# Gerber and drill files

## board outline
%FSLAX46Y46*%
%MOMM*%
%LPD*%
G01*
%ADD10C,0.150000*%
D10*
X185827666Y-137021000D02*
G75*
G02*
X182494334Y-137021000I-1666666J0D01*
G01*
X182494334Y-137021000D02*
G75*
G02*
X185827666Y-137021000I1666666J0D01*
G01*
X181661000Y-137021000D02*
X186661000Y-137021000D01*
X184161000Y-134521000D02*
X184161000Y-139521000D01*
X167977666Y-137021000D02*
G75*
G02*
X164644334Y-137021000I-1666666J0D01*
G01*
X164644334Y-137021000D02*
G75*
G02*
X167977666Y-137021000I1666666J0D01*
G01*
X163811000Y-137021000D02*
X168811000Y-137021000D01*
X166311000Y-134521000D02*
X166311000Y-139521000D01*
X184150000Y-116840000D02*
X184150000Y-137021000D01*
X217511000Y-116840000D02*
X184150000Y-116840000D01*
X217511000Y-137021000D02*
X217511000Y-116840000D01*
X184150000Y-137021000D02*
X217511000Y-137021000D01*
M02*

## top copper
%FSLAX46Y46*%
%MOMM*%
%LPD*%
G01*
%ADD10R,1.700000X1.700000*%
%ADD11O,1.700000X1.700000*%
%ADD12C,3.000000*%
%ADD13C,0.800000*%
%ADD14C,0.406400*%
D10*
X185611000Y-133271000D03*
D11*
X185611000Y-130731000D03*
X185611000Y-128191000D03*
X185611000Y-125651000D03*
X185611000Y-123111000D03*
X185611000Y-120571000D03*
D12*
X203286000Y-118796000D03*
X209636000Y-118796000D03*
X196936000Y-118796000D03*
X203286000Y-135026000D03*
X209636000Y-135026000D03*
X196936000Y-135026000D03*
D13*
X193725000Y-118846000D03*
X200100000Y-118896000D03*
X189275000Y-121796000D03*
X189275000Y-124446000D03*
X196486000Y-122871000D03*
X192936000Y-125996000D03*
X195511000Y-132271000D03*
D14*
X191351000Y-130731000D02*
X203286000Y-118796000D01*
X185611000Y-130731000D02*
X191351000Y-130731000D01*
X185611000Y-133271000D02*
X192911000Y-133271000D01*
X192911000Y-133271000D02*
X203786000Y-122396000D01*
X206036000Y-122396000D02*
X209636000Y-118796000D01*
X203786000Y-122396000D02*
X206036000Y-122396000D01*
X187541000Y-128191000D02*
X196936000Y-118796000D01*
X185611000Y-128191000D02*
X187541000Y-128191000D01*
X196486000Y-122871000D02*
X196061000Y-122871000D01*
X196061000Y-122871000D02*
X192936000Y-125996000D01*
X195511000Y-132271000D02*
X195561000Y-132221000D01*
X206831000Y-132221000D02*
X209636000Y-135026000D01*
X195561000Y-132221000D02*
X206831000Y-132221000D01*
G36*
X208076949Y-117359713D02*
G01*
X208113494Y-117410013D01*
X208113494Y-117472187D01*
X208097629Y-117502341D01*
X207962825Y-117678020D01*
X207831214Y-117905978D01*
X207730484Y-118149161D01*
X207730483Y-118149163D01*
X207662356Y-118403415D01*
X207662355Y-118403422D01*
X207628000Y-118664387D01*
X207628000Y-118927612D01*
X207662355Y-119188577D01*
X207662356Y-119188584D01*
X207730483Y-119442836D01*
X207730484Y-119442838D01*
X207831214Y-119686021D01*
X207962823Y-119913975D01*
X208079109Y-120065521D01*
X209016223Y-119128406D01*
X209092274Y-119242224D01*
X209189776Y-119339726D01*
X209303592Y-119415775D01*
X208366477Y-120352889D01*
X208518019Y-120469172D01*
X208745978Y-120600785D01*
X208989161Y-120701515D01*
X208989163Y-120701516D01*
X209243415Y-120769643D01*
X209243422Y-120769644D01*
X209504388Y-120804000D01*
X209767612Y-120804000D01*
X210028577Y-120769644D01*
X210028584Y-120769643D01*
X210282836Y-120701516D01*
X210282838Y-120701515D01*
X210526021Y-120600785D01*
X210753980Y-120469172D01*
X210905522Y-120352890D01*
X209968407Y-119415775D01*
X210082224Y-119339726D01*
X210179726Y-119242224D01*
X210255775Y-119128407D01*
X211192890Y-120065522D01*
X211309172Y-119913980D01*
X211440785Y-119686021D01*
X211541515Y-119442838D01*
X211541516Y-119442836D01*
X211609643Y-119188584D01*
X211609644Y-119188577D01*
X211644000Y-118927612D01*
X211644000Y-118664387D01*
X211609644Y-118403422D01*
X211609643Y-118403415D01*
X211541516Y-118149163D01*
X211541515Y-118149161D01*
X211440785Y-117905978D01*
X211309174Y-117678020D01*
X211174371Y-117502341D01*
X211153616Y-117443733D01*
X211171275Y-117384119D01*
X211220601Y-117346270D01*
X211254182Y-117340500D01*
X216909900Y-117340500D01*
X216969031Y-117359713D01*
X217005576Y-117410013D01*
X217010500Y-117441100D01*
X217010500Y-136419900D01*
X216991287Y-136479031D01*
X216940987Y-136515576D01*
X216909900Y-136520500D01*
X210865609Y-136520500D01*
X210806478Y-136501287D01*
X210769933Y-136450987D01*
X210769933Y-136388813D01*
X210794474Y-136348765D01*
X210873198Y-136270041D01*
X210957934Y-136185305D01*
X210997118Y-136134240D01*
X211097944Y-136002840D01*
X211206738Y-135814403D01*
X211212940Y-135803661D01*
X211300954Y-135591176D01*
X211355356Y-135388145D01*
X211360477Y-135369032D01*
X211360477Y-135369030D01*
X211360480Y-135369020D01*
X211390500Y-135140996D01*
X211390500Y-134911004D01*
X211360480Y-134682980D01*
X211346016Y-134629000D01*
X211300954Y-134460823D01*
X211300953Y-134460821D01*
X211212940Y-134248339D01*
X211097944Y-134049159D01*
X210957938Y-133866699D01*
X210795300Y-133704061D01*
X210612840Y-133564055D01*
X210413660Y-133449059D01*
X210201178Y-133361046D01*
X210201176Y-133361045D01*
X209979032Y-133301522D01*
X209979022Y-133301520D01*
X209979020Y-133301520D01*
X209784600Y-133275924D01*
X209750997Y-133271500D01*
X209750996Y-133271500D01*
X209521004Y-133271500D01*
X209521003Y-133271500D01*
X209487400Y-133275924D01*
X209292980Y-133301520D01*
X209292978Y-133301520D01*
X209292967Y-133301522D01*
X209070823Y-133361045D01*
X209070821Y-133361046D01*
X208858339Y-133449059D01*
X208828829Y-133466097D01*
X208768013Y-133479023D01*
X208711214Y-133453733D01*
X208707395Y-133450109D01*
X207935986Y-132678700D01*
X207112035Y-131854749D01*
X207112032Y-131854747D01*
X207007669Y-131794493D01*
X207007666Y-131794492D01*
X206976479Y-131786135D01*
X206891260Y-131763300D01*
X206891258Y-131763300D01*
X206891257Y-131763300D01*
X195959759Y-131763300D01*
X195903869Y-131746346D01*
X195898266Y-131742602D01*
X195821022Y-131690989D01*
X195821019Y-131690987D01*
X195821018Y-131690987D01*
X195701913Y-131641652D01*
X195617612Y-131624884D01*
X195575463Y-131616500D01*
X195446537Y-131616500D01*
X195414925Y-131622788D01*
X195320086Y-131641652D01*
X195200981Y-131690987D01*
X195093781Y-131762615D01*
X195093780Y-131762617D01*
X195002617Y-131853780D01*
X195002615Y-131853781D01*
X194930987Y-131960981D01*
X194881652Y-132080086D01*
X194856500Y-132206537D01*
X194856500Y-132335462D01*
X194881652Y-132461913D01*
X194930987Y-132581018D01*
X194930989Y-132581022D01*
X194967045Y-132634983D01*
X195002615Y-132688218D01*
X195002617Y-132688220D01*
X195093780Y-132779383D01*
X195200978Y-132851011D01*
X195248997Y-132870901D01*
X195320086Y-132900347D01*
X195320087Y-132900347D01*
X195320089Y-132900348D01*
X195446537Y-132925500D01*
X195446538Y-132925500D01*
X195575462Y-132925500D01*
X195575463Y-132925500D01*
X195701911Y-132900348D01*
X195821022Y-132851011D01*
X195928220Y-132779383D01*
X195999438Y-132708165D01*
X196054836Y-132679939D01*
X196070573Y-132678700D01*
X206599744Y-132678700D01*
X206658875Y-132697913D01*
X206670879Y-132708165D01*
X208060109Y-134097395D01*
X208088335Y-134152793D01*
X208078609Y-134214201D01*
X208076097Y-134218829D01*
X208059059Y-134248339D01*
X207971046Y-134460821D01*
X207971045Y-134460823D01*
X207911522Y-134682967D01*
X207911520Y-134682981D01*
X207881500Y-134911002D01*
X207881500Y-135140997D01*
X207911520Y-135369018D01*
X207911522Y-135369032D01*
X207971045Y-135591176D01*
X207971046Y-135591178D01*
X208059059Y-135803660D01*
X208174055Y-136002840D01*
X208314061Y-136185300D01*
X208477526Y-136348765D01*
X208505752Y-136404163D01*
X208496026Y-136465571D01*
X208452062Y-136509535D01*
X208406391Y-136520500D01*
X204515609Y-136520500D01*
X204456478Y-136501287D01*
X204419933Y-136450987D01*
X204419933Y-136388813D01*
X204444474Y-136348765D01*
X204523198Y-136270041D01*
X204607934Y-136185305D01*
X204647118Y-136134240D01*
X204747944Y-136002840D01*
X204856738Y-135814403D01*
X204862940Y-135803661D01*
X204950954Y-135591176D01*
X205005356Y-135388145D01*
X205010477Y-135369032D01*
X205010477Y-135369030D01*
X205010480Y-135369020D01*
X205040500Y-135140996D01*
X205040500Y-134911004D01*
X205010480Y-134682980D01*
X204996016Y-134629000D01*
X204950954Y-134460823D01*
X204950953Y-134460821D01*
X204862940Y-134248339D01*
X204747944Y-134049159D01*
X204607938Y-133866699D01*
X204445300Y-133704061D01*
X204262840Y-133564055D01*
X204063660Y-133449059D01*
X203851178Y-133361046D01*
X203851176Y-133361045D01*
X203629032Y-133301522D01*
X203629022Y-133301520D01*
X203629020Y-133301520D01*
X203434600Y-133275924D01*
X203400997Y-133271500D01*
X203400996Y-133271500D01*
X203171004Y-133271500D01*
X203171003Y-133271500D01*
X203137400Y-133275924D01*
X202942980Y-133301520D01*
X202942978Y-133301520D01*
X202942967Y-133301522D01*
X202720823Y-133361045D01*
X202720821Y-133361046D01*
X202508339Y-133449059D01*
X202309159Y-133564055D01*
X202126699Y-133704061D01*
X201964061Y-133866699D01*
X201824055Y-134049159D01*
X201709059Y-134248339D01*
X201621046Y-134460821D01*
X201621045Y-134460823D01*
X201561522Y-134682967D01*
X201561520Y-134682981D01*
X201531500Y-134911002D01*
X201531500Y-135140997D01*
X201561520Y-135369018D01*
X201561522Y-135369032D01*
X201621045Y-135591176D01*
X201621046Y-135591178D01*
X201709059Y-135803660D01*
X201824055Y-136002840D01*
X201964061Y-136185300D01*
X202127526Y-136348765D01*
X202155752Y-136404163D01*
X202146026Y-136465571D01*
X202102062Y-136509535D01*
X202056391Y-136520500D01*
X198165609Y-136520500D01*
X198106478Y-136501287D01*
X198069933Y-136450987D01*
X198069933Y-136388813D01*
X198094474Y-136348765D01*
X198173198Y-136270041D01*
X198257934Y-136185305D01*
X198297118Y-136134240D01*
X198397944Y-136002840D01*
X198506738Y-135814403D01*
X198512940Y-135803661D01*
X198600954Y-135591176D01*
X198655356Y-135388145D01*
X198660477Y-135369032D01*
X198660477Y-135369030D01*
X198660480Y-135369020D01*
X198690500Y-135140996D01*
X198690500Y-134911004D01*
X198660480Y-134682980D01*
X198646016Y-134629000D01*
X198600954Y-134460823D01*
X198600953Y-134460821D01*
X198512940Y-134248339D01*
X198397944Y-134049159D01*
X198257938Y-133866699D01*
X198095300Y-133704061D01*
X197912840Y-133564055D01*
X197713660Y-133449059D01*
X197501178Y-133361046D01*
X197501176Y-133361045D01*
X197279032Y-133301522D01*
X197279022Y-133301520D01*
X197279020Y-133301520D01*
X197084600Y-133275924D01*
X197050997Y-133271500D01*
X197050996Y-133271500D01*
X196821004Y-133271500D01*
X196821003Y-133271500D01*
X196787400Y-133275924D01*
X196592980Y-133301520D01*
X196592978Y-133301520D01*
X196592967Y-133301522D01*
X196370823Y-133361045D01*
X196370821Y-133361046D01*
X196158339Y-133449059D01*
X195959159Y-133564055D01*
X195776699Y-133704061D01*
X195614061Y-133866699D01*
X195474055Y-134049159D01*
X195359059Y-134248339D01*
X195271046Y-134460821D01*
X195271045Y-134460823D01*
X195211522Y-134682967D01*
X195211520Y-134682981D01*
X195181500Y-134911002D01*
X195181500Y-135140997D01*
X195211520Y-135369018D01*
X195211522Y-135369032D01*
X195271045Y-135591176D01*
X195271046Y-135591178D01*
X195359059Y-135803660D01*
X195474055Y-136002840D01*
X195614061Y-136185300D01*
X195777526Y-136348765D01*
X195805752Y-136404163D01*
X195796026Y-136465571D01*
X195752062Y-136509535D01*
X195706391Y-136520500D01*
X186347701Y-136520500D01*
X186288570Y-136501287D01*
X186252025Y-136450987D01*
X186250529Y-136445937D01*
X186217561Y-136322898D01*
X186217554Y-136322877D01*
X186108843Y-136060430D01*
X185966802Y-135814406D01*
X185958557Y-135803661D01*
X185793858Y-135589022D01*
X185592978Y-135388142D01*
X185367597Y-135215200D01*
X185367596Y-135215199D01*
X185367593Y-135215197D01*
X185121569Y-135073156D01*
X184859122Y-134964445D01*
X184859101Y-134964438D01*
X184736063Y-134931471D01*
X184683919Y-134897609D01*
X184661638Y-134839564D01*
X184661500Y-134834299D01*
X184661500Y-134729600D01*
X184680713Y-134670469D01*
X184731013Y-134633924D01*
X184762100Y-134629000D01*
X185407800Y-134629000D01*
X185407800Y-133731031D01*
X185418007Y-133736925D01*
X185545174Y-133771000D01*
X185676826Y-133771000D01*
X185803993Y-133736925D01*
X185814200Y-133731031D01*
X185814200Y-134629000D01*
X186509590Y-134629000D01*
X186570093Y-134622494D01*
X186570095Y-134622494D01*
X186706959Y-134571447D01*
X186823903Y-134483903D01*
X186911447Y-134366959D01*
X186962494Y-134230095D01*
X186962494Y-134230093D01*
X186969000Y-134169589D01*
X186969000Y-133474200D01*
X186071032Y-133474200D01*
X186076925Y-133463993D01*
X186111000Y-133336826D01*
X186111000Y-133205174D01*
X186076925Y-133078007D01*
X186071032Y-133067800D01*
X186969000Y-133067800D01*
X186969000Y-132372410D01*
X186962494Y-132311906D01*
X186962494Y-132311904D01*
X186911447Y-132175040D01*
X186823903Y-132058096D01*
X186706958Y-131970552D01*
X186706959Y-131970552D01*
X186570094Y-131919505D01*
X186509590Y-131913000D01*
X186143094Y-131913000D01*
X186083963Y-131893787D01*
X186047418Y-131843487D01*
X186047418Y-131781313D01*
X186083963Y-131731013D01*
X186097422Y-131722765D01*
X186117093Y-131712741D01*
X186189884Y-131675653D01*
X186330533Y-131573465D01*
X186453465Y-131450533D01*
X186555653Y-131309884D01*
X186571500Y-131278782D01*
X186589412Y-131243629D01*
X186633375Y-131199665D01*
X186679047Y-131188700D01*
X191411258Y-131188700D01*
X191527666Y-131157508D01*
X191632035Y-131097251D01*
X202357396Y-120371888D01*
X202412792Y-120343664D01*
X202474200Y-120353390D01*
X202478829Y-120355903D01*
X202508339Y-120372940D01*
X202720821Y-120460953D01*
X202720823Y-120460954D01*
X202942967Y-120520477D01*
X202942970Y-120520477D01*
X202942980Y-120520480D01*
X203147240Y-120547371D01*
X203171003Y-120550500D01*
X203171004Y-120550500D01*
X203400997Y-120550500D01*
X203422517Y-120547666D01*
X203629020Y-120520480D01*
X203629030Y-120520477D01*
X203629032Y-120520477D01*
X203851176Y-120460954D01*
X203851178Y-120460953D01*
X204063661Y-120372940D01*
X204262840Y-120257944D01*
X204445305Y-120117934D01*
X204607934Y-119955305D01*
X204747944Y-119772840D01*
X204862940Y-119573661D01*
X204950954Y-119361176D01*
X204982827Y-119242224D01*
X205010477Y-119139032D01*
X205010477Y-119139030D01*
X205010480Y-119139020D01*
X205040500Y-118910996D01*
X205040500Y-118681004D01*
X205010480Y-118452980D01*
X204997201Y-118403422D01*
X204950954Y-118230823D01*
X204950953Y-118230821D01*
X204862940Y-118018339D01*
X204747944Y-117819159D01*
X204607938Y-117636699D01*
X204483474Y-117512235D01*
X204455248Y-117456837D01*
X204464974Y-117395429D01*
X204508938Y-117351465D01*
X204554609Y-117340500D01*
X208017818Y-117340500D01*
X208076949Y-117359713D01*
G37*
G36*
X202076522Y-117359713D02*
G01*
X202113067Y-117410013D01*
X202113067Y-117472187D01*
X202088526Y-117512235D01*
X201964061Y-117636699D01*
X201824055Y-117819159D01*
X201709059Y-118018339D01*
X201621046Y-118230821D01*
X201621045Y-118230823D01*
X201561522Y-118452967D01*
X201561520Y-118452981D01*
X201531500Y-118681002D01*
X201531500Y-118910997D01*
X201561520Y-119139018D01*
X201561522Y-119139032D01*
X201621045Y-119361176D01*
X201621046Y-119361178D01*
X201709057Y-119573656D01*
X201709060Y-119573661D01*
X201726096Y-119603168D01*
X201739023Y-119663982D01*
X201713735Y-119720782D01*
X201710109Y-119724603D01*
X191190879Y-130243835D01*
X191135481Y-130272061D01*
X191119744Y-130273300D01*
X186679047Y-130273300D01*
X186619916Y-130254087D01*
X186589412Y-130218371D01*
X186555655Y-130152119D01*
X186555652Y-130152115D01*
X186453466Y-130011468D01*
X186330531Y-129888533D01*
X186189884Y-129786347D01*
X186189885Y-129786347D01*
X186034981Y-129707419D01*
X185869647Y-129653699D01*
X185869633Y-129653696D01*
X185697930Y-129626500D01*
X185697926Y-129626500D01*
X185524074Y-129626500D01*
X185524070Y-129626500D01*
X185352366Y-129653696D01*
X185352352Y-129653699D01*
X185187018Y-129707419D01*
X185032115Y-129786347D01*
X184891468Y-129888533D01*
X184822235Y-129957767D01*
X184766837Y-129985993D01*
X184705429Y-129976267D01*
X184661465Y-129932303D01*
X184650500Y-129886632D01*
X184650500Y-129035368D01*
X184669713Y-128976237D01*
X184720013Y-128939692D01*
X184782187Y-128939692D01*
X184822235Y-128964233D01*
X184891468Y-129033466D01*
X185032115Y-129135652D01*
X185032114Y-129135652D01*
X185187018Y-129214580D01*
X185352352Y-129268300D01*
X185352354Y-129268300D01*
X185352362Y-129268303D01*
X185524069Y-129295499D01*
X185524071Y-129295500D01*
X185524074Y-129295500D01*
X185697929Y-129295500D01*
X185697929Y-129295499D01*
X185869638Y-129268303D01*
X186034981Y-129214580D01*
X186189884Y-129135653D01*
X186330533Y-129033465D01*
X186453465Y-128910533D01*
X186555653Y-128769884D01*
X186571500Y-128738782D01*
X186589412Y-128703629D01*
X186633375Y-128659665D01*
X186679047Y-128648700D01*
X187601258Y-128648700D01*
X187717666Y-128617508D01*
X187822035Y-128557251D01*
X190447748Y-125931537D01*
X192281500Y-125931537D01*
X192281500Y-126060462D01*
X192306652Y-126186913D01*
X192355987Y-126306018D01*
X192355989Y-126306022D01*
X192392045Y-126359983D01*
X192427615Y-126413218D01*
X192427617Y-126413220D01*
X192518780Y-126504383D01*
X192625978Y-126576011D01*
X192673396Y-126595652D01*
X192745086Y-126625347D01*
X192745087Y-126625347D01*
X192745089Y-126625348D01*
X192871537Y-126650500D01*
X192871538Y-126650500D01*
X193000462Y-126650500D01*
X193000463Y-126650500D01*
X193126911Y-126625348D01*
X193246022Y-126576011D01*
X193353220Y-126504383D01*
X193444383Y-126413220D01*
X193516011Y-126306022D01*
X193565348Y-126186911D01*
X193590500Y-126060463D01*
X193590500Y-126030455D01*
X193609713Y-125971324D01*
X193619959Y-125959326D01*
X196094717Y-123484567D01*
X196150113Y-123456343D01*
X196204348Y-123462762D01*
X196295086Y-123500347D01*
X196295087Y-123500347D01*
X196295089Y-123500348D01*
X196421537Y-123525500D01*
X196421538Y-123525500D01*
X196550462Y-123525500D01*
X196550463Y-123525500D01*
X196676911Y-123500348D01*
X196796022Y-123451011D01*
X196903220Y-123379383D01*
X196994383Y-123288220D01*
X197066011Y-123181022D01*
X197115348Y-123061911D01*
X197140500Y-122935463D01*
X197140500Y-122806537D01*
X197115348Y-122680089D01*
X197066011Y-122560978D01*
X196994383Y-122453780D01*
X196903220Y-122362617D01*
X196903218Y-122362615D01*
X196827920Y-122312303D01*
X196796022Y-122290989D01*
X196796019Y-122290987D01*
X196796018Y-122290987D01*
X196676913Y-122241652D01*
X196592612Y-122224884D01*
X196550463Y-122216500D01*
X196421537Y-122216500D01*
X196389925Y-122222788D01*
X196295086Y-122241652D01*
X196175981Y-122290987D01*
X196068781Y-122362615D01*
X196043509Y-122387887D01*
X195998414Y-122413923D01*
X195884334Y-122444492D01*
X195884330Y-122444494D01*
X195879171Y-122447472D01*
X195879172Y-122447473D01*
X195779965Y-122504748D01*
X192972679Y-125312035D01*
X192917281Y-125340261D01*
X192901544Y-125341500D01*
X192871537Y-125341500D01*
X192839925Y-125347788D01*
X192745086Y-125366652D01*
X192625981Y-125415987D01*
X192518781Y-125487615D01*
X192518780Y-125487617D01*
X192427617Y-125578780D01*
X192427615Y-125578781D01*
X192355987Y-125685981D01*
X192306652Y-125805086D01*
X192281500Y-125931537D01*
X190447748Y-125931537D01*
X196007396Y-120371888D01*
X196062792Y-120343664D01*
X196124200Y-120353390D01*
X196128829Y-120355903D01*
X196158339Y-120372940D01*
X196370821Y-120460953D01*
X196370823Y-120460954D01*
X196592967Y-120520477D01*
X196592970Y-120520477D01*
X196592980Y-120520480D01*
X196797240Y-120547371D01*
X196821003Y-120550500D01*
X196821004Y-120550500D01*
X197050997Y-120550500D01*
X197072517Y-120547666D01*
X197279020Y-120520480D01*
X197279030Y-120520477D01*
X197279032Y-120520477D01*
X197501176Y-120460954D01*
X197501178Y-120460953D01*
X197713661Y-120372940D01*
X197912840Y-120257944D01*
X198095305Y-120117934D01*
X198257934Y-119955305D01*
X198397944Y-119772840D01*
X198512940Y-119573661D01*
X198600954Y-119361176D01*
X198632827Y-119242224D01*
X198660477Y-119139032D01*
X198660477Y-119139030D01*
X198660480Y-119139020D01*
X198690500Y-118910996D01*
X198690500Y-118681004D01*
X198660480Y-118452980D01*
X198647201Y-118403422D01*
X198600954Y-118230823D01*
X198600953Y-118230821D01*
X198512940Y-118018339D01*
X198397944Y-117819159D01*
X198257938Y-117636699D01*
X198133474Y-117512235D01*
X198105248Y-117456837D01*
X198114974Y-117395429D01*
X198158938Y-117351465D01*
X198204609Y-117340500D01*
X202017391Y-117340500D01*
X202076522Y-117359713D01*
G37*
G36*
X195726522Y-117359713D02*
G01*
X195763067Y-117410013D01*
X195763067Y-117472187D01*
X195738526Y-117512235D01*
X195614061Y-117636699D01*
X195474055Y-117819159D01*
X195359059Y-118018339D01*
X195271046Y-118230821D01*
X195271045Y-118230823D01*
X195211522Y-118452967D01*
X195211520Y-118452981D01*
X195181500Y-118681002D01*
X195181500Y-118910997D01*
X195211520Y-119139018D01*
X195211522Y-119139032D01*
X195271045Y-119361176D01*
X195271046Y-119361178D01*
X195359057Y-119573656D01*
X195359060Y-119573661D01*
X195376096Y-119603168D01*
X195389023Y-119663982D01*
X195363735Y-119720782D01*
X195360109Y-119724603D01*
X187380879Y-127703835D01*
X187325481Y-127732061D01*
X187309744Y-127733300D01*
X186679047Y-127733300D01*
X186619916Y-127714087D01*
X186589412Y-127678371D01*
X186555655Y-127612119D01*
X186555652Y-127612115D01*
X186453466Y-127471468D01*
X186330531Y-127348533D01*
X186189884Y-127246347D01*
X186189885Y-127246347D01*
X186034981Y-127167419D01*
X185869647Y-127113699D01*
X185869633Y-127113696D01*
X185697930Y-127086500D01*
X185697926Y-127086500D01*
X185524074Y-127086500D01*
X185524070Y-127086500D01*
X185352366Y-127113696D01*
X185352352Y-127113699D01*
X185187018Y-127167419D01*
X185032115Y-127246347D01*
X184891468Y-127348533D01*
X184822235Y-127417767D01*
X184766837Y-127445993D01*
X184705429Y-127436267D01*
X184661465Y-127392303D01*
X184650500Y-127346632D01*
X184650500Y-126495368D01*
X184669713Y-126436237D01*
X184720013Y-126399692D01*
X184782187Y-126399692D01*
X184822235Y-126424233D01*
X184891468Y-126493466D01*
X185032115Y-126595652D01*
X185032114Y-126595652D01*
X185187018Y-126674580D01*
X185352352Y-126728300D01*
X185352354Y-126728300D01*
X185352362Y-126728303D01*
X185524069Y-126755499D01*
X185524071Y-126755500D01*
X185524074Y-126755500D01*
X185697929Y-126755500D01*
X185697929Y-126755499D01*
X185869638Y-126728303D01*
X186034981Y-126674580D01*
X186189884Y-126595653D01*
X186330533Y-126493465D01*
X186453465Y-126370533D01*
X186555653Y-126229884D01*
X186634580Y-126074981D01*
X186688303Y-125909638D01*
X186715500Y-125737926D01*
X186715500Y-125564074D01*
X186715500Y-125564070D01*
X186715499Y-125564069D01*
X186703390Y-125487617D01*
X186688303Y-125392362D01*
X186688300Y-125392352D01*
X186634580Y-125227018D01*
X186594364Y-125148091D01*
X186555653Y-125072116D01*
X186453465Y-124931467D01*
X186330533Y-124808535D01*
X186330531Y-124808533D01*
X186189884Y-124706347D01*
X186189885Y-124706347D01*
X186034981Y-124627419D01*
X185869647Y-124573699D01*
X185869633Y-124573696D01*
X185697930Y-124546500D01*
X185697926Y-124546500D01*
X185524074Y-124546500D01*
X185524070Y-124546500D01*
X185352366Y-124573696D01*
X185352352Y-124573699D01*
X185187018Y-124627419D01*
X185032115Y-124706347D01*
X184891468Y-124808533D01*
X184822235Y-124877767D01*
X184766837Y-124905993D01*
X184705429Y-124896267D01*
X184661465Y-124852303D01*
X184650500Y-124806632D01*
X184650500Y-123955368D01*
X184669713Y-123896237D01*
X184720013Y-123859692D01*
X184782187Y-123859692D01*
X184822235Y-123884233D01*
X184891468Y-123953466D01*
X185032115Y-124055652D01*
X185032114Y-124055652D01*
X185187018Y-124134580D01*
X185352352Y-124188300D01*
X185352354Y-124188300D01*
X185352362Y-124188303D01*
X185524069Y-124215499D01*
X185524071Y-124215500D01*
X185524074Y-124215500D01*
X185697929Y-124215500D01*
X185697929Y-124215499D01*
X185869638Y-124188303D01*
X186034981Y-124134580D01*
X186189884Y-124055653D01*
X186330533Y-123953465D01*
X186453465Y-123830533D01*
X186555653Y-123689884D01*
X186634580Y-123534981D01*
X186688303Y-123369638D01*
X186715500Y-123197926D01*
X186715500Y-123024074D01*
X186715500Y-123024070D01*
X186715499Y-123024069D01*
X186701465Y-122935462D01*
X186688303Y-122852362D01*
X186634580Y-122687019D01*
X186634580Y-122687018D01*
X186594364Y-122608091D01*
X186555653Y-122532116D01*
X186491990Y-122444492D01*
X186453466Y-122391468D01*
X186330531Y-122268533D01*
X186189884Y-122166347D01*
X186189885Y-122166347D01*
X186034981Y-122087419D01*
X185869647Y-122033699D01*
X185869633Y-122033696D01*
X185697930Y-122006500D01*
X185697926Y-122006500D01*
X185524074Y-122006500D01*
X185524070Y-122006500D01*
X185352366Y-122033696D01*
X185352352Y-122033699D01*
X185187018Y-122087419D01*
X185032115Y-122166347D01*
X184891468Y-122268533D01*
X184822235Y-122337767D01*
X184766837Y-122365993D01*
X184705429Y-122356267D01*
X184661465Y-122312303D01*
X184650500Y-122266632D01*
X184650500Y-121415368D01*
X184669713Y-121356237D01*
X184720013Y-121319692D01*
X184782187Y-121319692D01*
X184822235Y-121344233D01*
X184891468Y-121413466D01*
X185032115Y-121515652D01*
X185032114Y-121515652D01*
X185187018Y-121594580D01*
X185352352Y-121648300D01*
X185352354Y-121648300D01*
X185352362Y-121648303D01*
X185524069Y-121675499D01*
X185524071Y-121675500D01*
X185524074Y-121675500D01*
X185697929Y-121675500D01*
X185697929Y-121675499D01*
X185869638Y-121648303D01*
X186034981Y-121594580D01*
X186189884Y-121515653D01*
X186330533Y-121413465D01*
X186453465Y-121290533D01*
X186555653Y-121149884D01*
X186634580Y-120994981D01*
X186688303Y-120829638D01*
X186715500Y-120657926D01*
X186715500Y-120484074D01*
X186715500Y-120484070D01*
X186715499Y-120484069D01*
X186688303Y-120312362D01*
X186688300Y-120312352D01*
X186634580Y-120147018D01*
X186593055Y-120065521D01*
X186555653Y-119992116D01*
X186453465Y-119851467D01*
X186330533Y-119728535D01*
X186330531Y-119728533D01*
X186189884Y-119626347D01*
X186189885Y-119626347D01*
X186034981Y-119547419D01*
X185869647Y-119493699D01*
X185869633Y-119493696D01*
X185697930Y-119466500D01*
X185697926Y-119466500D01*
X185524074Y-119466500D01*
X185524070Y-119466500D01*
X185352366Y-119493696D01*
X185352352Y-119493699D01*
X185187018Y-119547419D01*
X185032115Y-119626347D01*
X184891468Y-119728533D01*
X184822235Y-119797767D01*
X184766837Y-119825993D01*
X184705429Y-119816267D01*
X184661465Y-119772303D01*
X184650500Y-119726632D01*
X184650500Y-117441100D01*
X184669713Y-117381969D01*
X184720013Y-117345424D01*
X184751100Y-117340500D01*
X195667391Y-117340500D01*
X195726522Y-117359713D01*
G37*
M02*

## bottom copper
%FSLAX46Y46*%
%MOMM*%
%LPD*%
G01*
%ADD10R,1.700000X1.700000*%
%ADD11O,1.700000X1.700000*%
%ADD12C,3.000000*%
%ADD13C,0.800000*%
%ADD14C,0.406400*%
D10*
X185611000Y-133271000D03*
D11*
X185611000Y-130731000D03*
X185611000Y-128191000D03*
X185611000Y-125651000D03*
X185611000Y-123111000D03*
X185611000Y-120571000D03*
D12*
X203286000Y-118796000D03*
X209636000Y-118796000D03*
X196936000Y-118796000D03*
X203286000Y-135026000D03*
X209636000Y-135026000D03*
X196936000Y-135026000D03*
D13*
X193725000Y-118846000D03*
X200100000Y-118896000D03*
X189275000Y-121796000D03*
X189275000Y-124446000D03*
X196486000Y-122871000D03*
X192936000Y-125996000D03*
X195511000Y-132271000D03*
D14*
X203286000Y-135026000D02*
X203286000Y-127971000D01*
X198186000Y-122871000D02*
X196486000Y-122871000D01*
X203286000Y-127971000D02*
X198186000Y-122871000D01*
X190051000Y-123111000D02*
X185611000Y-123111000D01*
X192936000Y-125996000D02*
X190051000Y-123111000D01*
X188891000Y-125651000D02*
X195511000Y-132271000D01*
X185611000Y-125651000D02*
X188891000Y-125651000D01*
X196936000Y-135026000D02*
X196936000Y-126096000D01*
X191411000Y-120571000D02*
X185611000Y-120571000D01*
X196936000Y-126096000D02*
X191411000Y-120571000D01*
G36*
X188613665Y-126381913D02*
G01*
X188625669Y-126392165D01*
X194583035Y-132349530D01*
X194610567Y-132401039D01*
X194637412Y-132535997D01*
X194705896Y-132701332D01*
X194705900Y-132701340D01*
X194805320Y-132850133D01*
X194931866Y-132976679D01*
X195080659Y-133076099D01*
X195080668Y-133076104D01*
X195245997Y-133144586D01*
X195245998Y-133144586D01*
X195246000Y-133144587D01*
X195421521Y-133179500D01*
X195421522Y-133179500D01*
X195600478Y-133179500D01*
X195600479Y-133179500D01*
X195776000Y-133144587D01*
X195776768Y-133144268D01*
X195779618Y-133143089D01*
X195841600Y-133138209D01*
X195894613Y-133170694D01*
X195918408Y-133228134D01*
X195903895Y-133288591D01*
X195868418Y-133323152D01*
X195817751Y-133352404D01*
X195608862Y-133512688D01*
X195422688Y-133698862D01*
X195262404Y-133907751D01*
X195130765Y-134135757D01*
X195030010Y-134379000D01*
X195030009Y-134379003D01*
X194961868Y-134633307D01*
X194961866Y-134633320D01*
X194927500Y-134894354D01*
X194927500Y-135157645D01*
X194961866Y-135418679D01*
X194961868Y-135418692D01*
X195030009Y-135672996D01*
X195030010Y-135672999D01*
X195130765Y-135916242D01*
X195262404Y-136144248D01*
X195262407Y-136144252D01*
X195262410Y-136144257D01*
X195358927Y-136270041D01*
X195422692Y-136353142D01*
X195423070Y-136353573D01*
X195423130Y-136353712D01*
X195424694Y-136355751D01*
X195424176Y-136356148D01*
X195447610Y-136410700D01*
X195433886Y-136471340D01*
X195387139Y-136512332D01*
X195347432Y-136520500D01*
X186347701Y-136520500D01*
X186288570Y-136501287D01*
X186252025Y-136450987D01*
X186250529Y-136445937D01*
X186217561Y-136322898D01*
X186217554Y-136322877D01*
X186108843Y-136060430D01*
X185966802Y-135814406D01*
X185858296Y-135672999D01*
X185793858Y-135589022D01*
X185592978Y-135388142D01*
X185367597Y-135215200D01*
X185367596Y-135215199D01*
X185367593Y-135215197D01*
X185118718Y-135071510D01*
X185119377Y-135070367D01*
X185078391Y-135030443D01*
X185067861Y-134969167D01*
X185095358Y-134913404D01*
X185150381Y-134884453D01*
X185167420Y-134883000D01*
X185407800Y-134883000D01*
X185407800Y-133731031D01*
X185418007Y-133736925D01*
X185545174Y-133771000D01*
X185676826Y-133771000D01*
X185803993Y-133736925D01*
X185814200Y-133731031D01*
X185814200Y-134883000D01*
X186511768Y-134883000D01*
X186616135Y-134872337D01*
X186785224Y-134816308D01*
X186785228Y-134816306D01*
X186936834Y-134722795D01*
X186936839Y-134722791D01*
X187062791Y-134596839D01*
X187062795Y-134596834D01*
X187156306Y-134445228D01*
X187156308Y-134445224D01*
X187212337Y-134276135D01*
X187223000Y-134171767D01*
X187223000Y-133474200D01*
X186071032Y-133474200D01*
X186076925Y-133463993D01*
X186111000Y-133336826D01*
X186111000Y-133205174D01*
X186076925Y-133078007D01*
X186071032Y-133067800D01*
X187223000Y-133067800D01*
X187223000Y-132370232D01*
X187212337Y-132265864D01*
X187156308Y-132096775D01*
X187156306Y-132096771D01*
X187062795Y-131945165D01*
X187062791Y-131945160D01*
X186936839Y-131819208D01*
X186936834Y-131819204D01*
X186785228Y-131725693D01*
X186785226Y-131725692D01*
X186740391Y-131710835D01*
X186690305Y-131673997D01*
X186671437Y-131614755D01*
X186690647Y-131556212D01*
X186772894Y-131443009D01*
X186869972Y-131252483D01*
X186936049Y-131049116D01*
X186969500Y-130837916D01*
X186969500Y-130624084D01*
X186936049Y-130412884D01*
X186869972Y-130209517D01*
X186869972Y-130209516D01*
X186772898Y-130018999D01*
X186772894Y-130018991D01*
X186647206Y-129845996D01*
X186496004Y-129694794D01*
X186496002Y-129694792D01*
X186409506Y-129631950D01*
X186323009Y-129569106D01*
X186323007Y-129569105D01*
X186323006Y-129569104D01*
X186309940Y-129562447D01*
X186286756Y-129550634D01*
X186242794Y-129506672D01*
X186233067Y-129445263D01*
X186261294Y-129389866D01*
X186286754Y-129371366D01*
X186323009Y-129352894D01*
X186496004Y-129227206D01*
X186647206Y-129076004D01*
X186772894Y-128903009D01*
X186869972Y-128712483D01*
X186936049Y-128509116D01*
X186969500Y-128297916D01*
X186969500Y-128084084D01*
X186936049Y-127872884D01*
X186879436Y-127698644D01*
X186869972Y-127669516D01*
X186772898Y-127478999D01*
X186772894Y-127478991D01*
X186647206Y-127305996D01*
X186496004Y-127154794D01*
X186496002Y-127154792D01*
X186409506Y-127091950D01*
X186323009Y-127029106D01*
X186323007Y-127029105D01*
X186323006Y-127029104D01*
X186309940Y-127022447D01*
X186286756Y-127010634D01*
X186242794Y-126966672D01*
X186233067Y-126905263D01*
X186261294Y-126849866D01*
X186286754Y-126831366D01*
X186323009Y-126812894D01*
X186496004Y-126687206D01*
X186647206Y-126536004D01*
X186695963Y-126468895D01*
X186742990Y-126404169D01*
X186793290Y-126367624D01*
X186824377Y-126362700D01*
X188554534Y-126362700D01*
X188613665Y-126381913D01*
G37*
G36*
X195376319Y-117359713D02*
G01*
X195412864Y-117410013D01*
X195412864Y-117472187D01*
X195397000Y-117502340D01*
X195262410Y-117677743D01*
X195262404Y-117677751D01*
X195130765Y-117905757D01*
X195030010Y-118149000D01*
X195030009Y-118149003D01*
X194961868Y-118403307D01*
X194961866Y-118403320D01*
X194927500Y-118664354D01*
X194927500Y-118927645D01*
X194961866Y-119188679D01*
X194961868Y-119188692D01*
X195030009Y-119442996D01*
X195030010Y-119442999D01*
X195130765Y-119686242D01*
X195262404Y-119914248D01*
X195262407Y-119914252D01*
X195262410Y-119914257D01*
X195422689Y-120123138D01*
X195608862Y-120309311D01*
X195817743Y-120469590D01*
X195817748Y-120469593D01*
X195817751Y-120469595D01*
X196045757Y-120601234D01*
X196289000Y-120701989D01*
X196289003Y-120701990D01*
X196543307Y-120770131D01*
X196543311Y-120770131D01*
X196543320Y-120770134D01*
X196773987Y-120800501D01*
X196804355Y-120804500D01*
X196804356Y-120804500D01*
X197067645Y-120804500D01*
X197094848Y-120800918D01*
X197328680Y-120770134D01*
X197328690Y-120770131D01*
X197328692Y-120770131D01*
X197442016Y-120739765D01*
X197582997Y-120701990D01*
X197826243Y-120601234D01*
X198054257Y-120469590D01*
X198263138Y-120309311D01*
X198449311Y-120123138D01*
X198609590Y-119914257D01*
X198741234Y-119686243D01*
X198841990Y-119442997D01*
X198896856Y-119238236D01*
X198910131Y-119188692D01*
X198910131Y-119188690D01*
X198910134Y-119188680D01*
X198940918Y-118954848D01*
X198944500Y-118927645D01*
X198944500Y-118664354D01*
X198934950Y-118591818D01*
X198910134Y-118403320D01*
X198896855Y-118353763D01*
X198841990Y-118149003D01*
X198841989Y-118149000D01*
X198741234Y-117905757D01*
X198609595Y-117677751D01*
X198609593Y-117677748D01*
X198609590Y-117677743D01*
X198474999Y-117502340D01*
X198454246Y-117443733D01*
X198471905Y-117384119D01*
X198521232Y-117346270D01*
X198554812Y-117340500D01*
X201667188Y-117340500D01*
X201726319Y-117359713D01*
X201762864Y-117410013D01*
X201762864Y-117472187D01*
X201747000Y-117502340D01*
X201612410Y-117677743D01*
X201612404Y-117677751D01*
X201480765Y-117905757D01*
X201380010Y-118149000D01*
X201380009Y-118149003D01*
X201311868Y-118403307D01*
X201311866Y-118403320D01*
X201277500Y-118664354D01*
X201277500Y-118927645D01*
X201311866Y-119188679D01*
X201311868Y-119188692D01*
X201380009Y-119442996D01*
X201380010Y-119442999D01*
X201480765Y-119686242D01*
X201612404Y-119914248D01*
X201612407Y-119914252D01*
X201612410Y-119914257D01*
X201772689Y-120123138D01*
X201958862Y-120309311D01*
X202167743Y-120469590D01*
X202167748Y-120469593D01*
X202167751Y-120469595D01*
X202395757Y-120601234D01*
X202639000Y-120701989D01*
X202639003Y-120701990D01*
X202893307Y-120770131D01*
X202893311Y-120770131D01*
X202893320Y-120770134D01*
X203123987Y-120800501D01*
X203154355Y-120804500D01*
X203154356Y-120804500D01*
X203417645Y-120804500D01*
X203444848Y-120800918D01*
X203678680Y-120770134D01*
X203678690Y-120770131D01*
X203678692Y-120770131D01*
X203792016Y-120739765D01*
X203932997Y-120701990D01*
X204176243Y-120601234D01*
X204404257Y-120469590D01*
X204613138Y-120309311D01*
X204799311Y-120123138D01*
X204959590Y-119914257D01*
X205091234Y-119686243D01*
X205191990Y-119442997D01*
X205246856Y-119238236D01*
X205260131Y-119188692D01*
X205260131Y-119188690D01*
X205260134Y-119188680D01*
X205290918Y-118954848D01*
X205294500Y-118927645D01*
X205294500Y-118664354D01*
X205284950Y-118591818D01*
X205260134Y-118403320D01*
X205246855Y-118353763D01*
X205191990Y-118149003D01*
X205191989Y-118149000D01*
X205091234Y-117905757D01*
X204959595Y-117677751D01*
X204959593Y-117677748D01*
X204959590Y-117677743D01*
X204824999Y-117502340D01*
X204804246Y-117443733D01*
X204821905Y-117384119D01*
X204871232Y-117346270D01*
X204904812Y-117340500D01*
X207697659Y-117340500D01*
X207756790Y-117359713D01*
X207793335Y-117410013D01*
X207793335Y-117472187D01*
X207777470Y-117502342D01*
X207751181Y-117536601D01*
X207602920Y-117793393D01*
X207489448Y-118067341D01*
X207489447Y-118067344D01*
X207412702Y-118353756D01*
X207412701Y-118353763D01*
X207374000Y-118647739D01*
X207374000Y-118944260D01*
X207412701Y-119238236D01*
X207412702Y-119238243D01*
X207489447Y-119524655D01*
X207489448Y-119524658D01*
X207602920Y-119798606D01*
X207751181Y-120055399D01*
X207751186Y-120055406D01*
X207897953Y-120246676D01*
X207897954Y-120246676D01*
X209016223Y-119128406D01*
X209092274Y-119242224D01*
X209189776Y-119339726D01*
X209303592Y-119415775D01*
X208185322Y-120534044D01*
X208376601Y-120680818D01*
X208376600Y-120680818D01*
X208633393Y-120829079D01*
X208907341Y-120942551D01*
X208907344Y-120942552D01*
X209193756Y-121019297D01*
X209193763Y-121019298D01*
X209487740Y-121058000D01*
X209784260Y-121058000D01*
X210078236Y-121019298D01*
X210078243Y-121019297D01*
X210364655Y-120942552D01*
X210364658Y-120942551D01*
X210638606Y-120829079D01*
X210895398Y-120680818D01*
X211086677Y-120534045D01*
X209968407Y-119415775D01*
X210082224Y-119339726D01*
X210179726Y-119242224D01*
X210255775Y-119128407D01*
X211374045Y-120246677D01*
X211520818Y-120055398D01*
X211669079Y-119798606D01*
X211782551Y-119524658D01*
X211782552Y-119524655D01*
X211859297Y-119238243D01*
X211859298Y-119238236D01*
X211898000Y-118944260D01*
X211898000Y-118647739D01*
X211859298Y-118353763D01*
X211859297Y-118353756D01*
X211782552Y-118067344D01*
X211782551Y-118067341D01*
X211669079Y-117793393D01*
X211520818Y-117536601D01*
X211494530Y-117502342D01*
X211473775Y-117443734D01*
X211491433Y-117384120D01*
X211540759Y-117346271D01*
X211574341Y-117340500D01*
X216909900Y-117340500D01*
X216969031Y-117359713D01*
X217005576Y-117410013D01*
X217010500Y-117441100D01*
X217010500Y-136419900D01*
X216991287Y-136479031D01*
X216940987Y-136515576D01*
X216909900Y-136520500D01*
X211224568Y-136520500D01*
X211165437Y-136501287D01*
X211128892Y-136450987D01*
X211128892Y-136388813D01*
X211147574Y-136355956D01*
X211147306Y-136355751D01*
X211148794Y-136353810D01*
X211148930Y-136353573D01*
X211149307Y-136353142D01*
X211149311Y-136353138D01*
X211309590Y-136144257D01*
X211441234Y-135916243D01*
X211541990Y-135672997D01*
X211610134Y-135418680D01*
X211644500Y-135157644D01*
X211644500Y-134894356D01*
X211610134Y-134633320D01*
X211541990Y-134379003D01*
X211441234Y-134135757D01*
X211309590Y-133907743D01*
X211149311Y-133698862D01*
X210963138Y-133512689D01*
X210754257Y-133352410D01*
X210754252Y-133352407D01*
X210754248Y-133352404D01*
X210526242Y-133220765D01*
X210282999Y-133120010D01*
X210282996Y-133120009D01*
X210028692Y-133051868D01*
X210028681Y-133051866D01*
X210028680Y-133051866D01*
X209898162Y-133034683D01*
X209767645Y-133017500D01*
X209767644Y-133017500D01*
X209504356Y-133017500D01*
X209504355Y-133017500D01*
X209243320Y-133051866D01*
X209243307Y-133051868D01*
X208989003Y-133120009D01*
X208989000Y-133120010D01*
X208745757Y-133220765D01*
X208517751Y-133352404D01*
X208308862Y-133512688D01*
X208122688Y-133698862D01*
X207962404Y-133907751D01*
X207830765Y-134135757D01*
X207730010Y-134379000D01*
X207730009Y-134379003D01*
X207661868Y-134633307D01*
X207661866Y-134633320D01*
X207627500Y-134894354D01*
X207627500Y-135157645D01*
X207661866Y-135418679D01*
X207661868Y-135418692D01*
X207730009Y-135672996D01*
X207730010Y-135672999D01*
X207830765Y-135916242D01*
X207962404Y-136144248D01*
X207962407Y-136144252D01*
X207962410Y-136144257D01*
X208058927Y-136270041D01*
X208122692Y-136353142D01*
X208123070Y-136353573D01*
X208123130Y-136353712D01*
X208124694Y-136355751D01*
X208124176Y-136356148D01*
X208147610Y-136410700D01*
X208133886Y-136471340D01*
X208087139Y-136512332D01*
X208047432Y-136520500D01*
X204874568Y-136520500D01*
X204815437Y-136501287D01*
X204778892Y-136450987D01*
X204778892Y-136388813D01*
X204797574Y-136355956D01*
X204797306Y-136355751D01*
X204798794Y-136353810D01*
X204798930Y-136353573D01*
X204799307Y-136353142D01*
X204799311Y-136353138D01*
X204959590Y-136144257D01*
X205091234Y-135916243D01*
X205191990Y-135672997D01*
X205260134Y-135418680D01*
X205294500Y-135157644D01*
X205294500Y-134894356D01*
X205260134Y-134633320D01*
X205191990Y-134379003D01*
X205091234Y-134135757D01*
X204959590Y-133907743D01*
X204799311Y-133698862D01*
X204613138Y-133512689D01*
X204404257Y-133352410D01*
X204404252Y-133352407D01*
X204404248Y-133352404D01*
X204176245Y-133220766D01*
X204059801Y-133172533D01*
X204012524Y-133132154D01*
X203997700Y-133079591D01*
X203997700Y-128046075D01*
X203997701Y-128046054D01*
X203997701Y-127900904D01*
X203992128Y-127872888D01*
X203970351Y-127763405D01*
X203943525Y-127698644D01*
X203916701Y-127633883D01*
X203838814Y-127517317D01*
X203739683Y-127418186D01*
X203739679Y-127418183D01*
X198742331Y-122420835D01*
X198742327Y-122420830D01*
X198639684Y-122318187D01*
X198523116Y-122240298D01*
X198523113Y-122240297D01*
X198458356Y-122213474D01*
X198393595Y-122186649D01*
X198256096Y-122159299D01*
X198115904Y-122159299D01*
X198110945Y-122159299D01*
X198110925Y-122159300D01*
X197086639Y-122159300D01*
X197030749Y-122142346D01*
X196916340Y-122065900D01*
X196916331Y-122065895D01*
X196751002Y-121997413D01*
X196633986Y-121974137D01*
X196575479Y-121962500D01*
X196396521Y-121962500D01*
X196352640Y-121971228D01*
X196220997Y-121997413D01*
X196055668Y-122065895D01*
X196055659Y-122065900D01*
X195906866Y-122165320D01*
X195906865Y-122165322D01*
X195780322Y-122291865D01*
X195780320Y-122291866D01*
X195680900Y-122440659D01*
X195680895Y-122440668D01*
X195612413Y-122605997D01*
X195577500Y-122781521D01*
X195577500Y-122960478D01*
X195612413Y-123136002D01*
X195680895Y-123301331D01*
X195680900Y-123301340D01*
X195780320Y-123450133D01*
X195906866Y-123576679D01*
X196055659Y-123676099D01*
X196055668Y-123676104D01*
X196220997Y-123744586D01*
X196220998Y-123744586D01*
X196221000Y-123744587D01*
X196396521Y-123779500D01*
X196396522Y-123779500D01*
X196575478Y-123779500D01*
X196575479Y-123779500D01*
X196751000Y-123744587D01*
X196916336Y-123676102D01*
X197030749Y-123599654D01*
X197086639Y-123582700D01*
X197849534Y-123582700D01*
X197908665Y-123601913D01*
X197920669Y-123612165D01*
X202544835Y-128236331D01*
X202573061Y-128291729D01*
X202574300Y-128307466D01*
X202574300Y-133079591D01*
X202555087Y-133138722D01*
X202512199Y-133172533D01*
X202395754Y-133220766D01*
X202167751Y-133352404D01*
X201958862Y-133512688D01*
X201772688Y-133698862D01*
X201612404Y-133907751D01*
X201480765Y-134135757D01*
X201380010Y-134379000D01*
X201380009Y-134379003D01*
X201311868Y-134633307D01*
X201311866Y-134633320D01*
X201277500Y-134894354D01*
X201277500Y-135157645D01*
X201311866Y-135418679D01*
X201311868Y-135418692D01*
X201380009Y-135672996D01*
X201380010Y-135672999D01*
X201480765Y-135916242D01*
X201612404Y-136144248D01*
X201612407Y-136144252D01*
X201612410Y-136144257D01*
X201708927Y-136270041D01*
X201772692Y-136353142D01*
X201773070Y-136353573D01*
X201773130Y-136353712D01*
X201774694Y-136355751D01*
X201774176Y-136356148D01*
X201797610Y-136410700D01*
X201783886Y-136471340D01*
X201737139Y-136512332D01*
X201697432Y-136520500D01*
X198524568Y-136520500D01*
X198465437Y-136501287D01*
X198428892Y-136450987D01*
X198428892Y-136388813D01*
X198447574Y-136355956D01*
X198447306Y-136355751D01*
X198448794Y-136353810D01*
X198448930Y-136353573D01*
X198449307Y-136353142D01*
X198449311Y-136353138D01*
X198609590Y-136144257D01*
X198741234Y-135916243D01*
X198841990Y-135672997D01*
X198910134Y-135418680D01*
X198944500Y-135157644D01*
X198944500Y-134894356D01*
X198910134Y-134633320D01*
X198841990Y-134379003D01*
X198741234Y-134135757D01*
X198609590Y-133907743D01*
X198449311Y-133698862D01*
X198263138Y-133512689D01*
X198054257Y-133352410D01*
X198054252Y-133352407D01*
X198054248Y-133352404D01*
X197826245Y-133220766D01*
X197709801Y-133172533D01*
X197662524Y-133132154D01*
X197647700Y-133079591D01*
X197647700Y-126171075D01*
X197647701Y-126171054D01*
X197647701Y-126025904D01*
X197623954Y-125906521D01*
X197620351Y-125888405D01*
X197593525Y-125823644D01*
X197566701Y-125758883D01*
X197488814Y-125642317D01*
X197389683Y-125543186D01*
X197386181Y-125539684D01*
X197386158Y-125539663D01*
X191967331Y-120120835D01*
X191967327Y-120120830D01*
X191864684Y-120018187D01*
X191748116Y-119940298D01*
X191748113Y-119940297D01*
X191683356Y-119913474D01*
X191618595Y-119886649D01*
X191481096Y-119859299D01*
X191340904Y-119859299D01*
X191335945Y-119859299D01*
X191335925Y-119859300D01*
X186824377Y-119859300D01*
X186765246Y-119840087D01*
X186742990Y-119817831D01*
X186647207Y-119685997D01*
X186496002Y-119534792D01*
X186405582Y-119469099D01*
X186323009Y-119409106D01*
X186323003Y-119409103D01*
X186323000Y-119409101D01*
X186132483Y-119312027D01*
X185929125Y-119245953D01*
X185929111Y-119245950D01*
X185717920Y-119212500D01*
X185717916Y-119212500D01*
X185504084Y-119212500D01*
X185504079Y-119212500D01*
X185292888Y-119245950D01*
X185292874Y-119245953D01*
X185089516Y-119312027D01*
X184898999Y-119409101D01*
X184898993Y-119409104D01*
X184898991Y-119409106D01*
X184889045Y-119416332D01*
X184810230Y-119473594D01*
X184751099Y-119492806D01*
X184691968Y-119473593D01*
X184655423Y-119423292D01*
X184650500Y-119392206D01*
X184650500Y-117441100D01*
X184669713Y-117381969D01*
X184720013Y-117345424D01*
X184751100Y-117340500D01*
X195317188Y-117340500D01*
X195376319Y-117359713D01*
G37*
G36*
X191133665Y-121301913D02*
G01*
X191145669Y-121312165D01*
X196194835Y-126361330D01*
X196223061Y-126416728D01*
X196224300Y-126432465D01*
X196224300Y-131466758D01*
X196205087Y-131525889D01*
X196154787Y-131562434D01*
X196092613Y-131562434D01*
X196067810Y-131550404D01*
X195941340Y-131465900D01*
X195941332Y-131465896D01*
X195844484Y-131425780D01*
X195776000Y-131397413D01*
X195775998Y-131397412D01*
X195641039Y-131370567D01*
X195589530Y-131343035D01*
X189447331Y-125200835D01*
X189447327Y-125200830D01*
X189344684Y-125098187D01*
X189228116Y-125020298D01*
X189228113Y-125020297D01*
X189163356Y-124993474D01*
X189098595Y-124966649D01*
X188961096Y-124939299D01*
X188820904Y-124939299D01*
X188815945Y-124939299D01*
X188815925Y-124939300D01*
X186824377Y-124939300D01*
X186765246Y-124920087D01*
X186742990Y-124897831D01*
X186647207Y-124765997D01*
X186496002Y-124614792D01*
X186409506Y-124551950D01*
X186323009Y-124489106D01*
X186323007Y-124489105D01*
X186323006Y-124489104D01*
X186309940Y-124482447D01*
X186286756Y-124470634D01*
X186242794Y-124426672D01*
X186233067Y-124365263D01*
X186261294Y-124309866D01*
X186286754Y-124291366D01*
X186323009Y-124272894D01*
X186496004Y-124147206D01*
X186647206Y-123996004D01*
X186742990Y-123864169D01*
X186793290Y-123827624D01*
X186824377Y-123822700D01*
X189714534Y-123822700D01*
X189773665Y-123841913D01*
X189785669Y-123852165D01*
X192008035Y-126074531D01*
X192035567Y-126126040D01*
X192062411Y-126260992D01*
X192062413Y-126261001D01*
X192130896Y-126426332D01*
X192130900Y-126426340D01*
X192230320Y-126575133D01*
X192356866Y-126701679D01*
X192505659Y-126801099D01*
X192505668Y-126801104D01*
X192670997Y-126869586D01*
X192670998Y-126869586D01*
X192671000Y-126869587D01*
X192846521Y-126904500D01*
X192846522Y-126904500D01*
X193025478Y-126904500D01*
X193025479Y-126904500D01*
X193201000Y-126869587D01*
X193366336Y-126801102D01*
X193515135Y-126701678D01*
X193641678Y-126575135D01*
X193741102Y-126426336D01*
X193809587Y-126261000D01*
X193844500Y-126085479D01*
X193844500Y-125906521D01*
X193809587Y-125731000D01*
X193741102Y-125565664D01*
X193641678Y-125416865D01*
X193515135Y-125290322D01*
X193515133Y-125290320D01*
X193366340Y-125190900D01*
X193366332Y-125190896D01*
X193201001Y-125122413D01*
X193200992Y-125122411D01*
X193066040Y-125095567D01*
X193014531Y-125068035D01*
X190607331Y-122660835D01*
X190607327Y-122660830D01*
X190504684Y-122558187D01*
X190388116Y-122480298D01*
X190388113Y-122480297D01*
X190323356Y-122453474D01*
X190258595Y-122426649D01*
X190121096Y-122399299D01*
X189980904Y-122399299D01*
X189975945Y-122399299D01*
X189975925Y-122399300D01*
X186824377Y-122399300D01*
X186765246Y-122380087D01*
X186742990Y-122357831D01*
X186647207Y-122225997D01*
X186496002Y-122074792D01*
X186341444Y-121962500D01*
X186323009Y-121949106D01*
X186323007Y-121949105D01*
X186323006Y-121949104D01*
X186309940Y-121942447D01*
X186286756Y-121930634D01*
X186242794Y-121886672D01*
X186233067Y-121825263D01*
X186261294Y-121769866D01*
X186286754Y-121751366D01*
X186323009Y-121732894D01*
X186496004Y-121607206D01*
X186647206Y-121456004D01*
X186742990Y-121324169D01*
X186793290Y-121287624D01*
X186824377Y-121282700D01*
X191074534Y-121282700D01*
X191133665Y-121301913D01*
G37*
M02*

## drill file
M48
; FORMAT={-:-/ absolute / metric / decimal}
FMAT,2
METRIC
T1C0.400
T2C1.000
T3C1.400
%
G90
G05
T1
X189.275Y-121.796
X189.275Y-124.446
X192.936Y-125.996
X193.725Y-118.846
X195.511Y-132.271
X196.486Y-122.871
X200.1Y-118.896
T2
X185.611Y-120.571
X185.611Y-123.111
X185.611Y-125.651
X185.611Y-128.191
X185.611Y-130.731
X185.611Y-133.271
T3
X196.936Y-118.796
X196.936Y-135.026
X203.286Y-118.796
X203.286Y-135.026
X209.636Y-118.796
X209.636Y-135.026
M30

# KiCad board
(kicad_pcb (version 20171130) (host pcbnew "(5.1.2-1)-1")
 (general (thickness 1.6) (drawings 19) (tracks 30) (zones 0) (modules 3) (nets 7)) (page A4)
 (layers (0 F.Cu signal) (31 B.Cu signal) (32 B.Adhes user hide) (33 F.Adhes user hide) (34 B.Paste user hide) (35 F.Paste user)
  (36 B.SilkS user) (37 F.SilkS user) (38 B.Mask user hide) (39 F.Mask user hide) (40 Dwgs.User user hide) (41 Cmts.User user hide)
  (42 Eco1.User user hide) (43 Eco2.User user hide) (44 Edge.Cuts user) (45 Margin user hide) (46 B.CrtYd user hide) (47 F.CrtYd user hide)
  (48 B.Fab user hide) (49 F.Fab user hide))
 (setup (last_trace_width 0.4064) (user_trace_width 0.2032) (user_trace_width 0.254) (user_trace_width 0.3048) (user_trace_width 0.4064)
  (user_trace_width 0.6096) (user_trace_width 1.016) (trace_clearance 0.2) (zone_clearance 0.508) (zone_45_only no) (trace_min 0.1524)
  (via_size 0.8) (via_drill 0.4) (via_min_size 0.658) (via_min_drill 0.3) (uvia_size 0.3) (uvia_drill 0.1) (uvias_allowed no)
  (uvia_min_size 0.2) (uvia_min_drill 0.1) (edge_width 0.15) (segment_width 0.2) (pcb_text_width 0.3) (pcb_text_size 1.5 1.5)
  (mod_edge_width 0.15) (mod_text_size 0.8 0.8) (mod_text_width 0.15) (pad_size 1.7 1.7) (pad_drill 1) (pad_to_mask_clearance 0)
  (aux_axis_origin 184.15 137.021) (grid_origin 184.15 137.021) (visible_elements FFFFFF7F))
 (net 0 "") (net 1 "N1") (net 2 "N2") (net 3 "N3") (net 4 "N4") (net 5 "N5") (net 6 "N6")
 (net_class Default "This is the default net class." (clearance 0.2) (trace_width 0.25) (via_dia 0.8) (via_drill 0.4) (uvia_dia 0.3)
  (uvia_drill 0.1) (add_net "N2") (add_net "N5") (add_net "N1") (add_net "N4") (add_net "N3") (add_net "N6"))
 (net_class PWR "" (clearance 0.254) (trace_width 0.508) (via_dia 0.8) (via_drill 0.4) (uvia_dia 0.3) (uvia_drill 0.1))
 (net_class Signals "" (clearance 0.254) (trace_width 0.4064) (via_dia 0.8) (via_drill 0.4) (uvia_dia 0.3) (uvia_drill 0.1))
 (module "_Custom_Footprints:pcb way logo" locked (layer B.Cu) (at 202.436 128.296 180)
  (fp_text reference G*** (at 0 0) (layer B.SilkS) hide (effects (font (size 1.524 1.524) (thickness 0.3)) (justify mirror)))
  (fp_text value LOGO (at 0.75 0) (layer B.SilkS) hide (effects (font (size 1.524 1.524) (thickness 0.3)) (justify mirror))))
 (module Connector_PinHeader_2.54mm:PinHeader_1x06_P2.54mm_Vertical (layer F.Cu) (at 185.611 133.271 180)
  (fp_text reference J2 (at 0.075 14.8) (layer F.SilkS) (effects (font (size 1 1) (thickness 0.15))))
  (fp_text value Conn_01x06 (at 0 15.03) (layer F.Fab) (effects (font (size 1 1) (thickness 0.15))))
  (pad 1 thru_hole rect (at 0 0 180) (size 1.7 1.7) (drill 1) (layers *.Cu *.Mask) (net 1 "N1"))
  (pad 2 thru_hole oval (at 0 2.54 180) (size 1.7 1.7) (drill 1) (layers *.Cu *.Mask) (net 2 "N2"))
  (pad 3 thru_hole oval (at 0 5.08 180) (size 1.7 1.7) (drill 1) (layers *.Cu *.Mask) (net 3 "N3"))
  (pad 4 thru_hole oval (at 0 7.62 180) (size 1.7 1.7) (drill 1) (layers *.Cu *.Mask) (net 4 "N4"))
  (pad 5 thru_hole oval (at 0 10.16 180) (size 1.7 1.7) (drill 1) (layers *.Cu *.Mask) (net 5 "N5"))
  (pad 6 thru_hole oval (at 0 12.7 180) (size 1.7 1.7) (drill 1) (layers *.Cu *.Mask) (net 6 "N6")))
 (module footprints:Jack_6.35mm (layer F.Cu) (at 196.936 118.796)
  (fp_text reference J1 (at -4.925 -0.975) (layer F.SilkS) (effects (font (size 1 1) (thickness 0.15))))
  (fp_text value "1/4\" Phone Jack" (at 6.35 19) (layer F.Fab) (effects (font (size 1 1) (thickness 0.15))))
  (pad R thru_hole circle (at 6.35 0) (size 3 3) (drill 1.4) (layers *.Cu *.Mask) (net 2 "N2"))
  (pad S thru_hole circle (at 12.7 0) (size 3 3) (drill 1.4) (layers *.Cu *.Mask) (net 1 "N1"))
  (pad T thru_hole circle (at 0 0) (size 3 3) (drill 1.4) (layers *.Cu *.Mask) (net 3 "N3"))
  (pad RN thru_hole circle (at 6.35 16.23) (size 3 3) (drill 1.4) (layers *.Cu *.Mask) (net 5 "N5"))
  (pad SN thru_hole circle (at 12.7 16.23) (size 3 3) (drill 1.4) (layers *.Cu *.Mask) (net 4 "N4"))
  (pad TN thru_hole circle (at 0 16.23) (size 3 3) (drill 1.4) (layers *.Cu *.Mask) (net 6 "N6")))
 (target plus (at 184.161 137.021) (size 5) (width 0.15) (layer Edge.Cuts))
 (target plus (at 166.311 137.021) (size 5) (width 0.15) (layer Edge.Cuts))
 (gr_line (start 184.15 116.84) (end 184.15 137.021) (layer Edge.Cuts) (width 0.15))
 (gr_line (start 217.511 116.84) (end 184.15 116.84) (layer Edge.Cuts) (width 0.15))
 (gr_line (start 217.511 137.021) (end 217.511 116.84) (layer Edge.Cuts) (width 0.15))
 (gr_line (start 184.15 137.021) (end 217.511 137.021) (layer Edge.Cuts) (width 0.15))
 (segment (start 191.351 130.731) (end 203.286 118.796) (width 0.4064) (layer F.Cu) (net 2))
 (segment (start 185.611 130.731) (end 191.351 130.731) (width 0.4064) (layer F.Cu) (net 2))
 (segment (start 185.611 133.271) (end 192.911 133.271) (width 0.4064) (layer F.Cu) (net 1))
 (segment (start 192.911 133.271) (end 203.786 122.396) (width 0.4064) (layer F.Cu) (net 1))
 (segment (start 206.036 122.396) (end 209.636 118.796) (width 0.4064) (layer F.Cu) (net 1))
 (segment (start 203.786 122.396) (end 206.036 122.396) (width 0.4064) (layer F.Cu) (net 1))
 (via (at 193.725 118.846) (size 0.8) (drill 0.4) (layers F.Cu B.Cu) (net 1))
 (via (at 200.1 118.896) (size 0.8) (drill 0.4) (layers F.Cu B.Cu) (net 1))
 (via (at 189.275 121.796) (size 0.8) (drill 0.4) (layers F.Cu B.Cu) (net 1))
 (via (at 189.275 124.446) (size 0.8) (drill 0.4) (layers F.Cu B.Cu) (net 1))
 (segment (start 187.541 128.191) (end 196.936 118.796) (width 0.4064) (layer F.Cu) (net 3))
 (segment (start 185.611 128.191) (end 187.541 128.191) (width 0.4064) (layer F.Cu) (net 3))
 (segment (start 203.286 135.026) (end 203.286 127.971) (width 0.4064) (layer B.Cu) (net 5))
 (via (at 196.486 122.871) (size 0.8) (drill 0.4) (layers F.Cu B.Cu) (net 5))
 (segment (start 198.186 122.871) (end 196.486 122.871) (width 0.4064) (layer B.Cu) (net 5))
 (segment (start 203.286 127.971) (end 198.186 122.871) (width 0.4064) (layer B.Cu) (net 5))
 (segment (start 196.486 122.871) (end 196.061 122.871) (width 0.4064) (layer F.Cu) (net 5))
 (via (at 192.936 125.996) (size 0.8) (drill 0.4) (layers F.Cu B.Cu) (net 5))
 (segment (start 196.061 122.871) (end 192.936 125.996) (width 0.4064) (layer F.Cu) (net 5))
 (segment (start 190.051 123.111) (end 185.611 123.111) (width 0.4064) (layer B.Cu) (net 5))
 (segment (start 192.936 125.996) (end 190.051 123.111) (width 0.4064) (layer B.Cu) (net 5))
 (via (at 195.511 132.271) (size 0.8) (drill 0.4) (layers F.Cu B.Cu) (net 4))
 (segment (start 188.891 125.651) (end 195.511 132.271) (width 0.4064) (layer B.Cu) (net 4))
 (segment (start 185.611 125.651) (end 188.891 125.651) (width 0.4064) (layer B.Cu) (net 4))
 (segment (start 195.511 132.271) (end 195.561 132.221) (width 0.4064) (layer F.Cu) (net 4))
 (segment (start 206.831 132.221) (end 209.636 135.026) (width 0.4064) (layer F.Cu) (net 4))
 (segment (start 195.561 132.221) (end 206.831 132.221) (width 0.4064) (layer F.Cu) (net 4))
 (segment (start 196.936 135.026) (end 196.936 126.096) (width 0.4064) (layer B.Cu) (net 6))
 (segment (start 191.411 120.571) (end 185.611 120.571) (width 0.4064) (layer B.Cu) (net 6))
 (segment (start 196.936 126.096) (end 191.411 120.571) (width 0.4064) (layer B.Cu) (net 6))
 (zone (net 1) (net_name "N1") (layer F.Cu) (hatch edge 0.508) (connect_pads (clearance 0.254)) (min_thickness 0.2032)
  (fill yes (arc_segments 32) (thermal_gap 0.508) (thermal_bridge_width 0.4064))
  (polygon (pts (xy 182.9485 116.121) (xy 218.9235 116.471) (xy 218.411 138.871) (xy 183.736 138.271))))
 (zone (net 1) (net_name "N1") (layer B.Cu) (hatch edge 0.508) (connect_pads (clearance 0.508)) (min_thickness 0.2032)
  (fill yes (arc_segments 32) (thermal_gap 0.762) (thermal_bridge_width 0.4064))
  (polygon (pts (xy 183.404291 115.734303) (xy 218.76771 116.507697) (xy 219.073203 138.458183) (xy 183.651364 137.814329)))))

